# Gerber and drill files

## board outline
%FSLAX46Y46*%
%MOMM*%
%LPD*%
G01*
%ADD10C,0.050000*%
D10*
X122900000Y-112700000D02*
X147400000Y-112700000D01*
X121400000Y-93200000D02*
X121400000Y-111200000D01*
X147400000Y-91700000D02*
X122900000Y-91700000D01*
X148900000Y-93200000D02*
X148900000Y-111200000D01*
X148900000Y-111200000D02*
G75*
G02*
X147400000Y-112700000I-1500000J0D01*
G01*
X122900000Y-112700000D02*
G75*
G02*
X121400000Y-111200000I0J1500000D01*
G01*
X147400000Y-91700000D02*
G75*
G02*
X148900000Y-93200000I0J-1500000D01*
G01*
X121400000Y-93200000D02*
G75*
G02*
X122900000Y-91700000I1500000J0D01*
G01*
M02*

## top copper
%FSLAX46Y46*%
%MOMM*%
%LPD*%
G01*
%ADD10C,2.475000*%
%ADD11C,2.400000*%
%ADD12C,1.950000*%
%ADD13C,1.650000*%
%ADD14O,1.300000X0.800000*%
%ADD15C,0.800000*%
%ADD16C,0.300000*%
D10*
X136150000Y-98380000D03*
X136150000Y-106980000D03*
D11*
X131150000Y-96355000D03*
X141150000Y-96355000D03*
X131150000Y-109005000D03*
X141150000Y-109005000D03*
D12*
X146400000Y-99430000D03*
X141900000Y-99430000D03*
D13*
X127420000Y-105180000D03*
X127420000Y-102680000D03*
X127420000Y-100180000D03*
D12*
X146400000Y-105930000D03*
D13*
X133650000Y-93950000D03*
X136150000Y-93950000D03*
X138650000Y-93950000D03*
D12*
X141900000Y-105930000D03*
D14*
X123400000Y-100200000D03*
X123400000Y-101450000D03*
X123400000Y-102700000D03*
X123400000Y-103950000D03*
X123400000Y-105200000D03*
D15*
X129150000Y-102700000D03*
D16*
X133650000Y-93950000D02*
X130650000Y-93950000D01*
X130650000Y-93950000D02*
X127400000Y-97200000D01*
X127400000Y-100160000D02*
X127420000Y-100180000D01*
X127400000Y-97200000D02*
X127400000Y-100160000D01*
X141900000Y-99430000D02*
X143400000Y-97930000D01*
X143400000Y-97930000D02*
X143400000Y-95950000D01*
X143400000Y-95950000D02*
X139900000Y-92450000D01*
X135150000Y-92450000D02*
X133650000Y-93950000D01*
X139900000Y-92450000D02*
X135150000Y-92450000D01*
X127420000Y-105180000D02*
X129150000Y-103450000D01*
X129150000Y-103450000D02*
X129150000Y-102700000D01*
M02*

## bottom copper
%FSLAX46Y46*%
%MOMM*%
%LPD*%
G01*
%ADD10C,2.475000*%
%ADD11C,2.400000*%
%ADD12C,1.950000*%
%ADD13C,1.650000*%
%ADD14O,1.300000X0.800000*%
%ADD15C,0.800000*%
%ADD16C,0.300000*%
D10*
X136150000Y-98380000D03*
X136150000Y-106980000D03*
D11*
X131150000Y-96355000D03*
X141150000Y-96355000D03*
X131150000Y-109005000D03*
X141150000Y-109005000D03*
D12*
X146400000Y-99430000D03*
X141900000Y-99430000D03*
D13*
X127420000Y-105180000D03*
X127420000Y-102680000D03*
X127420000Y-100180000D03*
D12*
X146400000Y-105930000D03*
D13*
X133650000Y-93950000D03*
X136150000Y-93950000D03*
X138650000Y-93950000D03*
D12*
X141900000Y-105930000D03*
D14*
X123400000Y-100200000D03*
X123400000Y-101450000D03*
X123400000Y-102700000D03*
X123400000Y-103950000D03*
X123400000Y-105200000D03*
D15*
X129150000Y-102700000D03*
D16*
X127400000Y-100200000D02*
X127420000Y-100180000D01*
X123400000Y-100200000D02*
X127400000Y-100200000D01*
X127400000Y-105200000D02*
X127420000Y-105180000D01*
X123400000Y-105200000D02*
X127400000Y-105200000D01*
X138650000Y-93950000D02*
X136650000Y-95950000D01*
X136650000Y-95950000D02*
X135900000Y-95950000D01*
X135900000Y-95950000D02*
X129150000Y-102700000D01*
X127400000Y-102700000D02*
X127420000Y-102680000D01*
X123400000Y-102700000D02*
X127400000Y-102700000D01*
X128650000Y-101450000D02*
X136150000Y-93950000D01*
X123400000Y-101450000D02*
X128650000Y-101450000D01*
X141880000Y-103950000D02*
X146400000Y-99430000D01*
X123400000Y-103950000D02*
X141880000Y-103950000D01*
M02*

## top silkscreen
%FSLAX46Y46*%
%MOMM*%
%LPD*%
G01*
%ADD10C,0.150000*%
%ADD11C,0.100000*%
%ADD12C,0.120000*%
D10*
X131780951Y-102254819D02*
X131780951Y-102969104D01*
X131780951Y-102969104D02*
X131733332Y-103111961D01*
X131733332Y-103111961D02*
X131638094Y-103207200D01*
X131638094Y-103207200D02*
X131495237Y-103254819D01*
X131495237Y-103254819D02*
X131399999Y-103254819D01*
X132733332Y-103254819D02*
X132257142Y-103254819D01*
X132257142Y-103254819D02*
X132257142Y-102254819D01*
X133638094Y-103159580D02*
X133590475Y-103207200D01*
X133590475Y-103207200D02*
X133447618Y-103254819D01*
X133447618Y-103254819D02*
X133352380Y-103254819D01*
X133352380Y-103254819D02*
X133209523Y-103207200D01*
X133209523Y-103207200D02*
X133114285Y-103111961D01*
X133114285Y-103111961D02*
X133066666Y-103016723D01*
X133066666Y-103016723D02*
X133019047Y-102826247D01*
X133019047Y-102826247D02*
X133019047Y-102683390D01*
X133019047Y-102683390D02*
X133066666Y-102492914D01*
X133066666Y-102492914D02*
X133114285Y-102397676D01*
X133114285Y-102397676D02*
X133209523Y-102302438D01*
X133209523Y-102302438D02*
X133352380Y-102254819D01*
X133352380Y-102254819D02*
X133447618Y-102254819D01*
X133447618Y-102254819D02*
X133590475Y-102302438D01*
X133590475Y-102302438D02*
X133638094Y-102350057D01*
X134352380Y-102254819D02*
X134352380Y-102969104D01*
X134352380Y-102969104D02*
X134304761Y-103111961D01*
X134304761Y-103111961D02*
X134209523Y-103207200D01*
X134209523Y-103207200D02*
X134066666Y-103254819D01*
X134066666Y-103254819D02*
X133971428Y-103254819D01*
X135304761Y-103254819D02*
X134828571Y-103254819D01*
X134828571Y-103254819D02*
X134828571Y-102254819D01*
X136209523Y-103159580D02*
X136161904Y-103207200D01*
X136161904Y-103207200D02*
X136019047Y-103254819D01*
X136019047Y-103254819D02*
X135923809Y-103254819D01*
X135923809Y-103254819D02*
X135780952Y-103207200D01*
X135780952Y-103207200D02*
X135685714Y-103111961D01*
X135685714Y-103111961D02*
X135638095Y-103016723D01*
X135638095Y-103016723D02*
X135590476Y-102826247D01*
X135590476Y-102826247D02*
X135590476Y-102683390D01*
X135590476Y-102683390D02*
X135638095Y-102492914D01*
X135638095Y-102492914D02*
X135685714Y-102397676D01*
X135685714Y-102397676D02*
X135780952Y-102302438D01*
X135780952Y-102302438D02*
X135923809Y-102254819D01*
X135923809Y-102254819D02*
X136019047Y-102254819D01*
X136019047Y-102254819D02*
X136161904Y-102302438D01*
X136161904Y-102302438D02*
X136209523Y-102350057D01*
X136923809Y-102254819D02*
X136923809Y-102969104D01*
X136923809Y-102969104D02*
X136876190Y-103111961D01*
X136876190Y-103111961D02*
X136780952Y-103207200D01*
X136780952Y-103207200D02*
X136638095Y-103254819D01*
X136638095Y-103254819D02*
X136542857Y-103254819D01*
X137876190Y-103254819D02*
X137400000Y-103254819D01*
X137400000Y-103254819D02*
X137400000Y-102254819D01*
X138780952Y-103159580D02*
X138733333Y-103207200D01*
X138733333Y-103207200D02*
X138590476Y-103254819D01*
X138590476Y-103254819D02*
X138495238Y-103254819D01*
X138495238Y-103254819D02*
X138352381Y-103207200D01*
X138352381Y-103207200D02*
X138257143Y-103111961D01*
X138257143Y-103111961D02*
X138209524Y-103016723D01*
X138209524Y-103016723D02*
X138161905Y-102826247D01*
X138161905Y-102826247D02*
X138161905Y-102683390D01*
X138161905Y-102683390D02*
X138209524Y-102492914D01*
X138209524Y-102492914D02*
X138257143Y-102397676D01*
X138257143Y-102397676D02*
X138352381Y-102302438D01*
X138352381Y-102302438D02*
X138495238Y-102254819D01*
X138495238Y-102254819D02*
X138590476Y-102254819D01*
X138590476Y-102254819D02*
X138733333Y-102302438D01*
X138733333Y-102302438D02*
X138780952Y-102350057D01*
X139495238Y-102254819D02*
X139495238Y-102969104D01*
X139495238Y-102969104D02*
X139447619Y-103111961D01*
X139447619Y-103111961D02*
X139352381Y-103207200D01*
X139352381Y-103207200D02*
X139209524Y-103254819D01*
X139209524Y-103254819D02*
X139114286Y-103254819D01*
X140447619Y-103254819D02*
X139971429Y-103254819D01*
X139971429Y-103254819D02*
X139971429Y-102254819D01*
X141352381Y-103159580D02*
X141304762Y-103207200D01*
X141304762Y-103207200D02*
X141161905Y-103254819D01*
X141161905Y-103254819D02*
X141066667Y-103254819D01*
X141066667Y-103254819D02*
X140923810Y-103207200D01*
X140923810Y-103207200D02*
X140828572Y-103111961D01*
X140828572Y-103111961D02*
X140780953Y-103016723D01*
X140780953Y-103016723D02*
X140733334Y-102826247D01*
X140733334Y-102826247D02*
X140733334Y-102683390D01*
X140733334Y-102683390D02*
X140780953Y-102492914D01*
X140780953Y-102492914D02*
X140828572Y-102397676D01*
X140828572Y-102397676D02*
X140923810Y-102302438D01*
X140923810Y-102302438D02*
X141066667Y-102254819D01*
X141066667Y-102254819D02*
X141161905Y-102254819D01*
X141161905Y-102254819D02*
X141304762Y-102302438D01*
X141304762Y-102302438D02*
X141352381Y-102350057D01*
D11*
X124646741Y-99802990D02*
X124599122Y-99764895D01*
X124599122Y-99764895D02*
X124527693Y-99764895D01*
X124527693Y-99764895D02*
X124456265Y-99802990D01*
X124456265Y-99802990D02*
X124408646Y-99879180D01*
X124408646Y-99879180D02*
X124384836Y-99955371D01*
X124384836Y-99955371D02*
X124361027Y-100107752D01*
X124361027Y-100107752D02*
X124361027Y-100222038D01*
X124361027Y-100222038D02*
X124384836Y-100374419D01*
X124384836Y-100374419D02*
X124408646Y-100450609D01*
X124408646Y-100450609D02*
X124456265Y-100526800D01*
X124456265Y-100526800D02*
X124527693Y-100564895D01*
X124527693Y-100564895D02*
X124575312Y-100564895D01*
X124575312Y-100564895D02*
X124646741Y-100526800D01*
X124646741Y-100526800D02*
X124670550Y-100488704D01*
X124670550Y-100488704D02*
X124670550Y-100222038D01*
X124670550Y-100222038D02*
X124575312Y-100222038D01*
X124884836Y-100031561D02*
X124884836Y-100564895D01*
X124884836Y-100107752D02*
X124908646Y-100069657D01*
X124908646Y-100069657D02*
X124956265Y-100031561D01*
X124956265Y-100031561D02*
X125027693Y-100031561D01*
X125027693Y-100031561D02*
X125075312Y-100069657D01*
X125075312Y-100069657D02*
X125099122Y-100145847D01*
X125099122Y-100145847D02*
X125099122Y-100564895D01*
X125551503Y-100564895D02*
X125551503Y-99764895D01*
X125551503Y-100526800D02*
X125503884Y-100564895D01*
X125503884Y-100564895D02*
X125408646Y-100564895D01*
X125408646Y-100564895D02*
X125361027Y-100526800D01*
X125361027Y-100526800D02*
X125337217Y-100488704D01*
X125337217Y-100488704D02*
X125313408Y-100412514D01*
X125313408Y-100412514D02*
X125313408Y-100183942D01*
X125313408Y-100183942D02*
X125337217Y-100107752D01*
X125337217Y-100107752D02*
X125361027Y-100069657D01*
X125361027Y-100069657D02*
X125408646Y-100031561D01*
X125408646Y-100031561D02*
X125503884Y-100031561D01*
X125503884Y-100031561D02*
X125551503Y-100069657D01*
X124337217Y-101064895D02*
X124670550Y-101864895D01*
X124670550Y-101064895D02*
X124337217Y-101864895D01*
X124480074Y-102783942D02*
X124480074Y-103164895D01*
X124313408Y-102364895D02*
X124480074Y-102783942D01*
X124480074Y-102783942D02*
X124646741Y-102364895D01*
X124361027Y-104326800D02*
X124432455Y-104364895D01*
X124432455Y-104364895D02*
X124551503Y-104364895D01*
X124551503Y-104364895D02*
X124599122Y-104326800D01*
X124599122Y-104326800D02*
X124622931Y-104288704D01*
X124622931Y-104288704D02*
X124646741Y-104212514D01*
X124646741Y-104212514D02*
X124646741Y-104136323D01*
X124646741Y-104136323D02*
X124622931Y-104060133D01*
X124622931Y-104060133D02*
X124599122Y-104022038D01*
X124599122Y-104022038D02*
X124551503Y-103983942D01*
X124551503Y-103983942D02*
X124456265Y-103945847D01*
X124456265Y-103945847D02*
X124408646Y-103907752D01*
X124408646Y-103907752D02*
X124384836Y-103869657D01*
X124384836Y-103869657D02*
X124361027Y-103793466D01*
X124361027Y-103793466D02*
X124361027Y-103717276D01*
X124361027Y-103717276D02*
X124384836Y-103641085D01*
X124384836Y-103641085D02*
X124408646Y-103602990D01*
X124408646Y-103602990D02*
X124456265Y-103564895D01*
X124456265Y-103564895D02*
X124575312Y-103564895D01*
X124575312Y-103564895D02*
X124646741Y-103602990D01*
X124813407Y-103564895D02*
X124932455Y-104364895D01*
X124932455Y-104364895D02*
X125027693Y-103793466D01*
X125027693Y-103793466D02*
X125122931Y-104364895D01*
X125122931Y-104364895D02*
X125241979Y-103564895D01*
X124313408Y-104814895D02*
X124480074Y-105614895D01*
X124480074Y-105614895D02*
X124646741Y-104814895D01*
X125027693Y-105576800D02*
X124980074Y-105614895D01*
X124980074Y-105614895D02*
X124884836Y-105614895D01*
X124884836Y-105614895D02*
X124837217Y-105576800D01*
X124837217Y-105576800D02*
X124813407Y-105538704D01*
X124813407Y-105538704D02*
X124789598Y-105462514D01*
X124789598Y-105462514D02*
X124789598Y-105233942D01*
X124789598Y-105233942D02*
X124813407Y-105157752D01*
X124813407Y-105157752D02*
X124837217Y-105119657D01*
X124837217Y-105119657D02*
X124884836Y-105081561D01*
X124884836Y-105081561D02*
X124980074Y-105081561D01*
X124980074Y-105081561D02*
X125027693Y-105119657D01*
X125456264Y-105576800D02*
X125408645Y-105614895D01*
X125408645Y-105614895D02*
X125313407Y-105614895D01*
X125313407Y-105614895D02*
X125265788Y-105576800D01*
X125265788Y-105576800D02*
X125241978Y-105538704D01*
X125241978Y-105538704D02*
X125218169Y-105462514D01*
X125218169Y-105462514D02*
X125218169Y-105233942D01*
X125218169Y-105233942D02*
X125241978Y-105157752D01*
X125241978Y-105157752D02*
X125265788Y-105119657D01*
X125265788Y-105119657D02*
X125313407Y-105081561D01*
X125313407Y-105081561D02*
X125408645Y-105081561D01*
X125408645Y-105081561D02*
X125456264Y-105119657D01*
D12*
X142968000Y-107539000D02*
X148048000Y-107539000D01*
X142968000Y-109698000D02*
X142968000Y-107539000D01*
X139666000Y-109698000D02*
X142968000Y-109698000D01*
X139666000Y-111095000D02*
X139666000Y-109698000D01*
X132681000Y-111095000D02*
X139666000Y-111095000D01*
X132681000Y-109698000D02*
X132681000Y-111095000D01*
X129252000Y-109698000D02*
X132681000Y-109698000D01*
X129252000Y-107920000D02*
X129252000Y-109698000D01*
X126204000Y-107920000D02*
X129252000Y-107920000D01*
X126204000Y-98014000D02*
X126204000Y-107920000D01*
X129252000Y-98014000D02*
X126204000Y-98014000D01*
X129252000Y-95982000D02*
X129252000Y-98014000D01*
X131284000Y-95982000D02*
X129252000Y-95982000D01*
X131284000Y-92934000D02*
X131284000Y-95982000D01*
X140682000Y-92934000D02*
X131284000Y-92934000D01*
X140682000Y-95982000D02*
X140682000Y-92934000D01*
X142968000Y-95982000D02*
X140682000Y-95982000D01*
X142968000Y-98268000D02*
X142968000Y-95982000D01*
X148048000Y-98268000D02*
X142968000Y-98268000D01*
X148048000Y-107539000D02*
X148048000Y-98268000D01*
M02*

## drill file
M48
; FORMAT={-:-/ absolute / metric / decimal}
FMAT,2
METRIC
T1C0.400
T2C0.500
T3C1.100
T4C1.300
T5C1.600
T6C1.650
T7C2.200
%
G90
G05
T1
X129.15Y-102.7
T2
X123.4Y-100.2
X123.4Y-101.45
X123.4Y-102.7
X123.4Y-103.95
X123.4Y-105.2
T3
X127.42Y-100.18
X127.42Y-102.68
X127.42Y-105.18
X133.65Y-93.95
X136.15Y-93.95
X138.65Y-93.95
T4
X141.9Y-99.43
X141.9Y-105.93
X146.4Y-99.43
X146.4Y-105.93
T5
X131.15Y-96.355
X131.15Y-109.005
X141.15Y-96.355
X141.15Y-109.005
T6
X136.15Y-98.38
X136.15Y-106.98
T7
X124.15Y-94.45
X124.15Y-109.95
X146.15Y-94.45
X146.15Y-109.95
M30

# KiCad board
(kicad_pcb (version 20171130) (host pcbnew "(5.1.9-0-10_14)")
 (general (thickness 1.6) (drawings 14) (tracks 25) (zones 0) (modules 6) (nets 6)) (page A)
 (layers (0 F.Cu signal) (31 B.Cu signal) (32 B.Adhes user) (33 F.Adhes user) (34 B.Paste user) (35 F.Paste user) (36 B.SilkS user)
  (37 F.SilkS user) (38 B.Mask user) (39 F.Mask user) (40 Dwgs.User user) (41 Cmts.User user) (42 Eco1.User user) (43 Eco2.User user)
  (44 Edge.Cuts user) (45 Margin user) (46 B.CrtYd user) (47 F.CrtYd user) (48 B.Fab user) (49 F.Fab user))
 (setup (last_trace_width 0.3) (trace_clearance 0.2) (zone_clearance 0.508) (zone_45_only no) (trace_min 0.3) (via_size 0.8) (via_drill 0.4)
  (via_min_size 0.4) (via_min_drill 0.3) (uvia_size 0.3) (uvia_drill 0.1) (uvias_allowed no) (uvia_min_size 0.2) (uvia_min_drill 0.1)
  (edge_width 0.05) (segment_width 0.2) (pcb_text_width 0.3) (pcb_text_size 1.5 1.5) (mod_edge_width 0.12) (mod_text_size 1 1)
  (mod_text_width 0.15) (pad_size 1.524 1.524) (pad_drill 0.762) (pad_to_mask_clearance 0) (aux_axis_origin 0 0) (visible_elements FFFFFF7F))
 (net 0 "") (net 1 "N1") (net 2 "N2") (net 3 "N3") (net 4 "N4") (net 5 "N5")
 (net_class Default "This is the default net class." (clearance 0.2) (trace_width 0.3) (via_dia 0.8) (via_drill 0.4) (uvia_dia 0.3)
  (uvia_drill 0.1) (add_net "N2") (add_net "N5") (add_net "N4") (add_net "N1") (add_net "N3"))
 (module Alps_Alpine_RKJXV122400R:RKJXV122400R (layer F.Cu) (at 138.65 93.95 90)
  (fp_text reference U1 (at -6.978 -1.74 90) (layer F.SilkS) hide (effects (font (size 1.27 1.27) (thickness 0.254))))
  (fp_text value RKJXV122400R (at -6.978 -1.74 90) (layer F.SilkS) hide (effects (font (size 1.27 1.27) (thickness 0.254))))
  (fp_line (start -13.589 4.318) (end -13.589 9.398) (layer F.SilkS) (width 0.12))
  (fp_line (start -15.748 4.318) (end -13.589 4.318) (layer F.SilkS) (width 0.12))
  (fp_line (start -15.748 1.016) (end -15.748 4.318) (layer F.SilkS) (width 0.12))
  (fp_line (start -17.145 1.016) (end -15.748 1.016) (layer F.SilkS) (width 0.12))
  (fp_line (start -17.145 -5.969) (end -17.145 1.016) (layer F.SilkS) (width 0.12))
  (fp_line (start -15.748 -5.969) (end -17.145 -5.969) (layer F.SilkS) (width 0.12))
  (fp_line (start -15.748 -9.398) (end -15.748 -5.969) (layer F.SilkS) (width 0.12))
  (fp_line (start -13.97 -9.398) (end -15.748 -9.398) (layer F.SilkS) (width 0.12))
  (fp_line (start -13.97 -12.446) (end -13.97 -9.398) (layer F.SilkS) (width 0.12))
  (fp_line (start -4.064 -12.446) (end -13.97 -12.446) (layer F.SilkS) (width 0.12))
  (fp_line (start -4.064 -9.398) (end -4.064 -12.446) (layer F.SilkS) (width 0.12))
  (fp_line (start -2.032 -9.398) (end -4.064 -9.398) (layer F.SilkS) (width 0.12))
  (fp_line (start -2.032 -7.366) (end -2.032 -9.398) (layer F.SilkS) (width 0.12))
  (fp_line (start 1.016 -7.366) (end -2.032 -7.366) (layer F.SilkS) (width 0.12))
  (fp_line (start 1.016 2.032) (end 1.016 -7.366) (layer F.SilkS) (width 0.12))
  (fp_line (start -2.032 2.032) (end 1.016 2.032) (layer F.SilkS) (width 0.12))
  (fp_line (start -2.032 4.318) (end -2.032 2.032) (layer F.SilkS) (width 0.12))
  (fp_line (start -4.318 4.318) (end -2.032 4.318) (layer F.SilkS) (width 0.12))
  (fp_line (start -4.318 9.398) (end -4.318 4.318) (layer F.SilkS) (width 0.12))
  (fp_line (start -13.589 9.398) (end -4.318 9.398) (layer F.SilkS) (width 0.12))
  (pad MH6 thru_hole circle (at -4.43 -2.5 90) (size 2.475 2.475) (drill 1.65) (layers *.Cu *.Mask))
  (pad MH5 thru_hole circle (at -13.03 -2.5 90) (size 2.475 2.475) (drill 1.65) (layers *.Cu *.Mask))
  (pad MH4 thru_hole circle (at -2.405 -7.5 90) (size 2.4 2.4) (drill 1.6) (layers *.Cu *.Mask))
  (pad MH3 thru_hole circle (at -2.405 2.5 90) (size 2.4 2.4) (drill 1.6) (layers *.Cu *.Mask))
  (pad MH2 thru_hole circle (at -15.055 -7.5 90) (size 2.4 2.4) (drill 1.6) (layers *.Cu *.Mask))
  (pad MH1 thru_hole circle (at -15.055 2.5 90) (size 2.4 2.4) (drill 1.6) (layers *.Cu *.Mask))
  (pad D1 thru_hole circle (at -5.48 7.75 90) (size 1.95 1.95) (drill 1.3) (layers *.Cu *.Mask) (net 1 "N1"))
  (pad C1 thru_hole circle (at -5.48 3.25 90) (size 1.95 1.95) (drill 1.3) (layers *.Cu *.Mask) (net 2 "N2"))
  (pad B13 thru_hole circle (at -11.23 -11.23 90) (size 1.65 1.65) (drill 1.1) (layers *.Cu *.Mask) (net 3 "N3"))
  (pad B12 thru_hole circle (at -8.73 -11.23 90) (size 1.65 1.65) (drill 1.1) (layers *.Cu *.Mask) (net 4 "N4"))
  (pad B11 thru_hole circle (at -6.23 -11.23 90) (size 1.65 1.65) (drill 1.1) (layers *.Cu *.Mask) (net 2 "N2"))
  (pad B1 thru_hole circle (at -11.98 7.75 90) (size 1.95 1.95) (drill 1.3) (layers *.Cu *.Mask))
  (pad A13 thru_hole circle (at 0 -5 90) (size 1.65 1.65) (drill 1.1) (layers *.Cu *.Mask) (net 2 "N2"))
  (pad A12 thru_hole circle (at 0 -2.5 90) (size 1.65 1.65) (drill 1.1) (layers *.Cu *.Mask) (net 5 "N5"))
  (pad A11 thru_hole circle (at 0 0 90) (size 1.65 1.65) (drill 1.1) (layers *.Cu *.Mask) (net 3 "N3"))
  (pad A1 thru_hole circle (at -11.98 3.25 90) (size 1.95 1.95) (drill 1.3) (layers *.Cu *.Mask)))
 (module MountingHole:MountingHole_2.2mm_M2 (layer F.Cu) (at 146.15 109.95)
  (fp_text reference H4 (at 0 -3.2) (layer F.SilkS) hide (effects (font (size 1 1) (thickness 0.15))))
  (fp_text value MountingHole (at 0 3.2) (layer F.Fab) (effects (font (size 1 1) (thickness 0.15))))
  (pad 1 np_thru_hole circle (at 0 0) (size 2.2 2.2) (drill 2.2) (layers *.Cu *.Mask)))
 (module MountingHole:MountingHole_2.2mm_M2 (layer F.Cu) (at 146.15 94.45)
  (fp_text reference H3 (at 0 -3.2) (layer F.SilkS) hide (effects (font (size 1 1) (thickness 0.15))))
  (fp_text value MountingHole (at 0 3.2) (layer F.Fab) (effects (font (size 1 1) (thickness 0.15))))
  (pad 1 np_thru_hole circle (at 0 0) (size 2.2 2.2) (drill 2.2) (layers *.Cu *.Mask)))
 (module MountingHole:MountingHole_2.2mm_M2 (layer F.Cu) (at 124.15 109.95)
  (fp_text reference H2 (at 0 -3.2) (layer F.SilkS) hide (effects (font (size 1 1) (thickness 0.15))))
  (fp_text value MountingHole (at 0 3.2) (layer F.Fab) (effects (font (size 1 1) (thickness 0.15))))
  (pad 1 np_thru_hole circle (at 0 0) (size 2.2 2.2) (drill 2.2) (layers *.Cu *.Mask)))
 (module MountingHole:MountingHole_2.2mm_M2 (layer F.Cu) (at 124.15 94.45)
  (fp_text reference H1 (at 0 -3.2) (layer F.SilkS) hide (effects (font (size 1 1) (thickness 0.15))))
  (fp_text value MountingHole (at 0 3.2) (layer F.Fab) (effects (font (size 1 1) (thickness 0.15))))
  (pad 1 np_thru_hole circle (at 0 0) (size 2.2 2.2) (drill 2.2) (layers *.Cu *.Mask)))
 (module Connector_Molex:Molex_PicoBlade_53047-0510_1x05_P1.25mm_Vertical (layer B.Cu) (at 123.4 100.2 270)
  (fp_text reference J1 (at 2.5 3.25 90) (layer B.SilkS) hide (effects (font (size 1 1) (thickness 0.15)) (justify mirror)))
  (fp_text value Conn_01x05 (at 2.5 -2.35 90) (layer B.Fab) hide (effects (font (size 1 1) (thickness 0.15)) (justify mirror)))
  (pad 1 thru_hole oval (at 0 0 270) (size 0.8 1.3) (drill 0.5) (layers *.Cu *.Mask) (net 2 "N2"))
  (pad 2 thru_hole oval (at 1.25 0 270) (size 0.8 1.3) (drill 0.5) (layers *.Cu *.Mask) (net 5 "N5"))
  (pad 3 thru_hole oval (at 2.5 0 270) (size 0.8 1.3) (drill 0.5) (layers *.Cu *.Mask) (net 4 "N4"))
  (pad 4 thru_hole oval (at 3.75 0 270) (size 0.8 1.3) (drill 0.5) (layers *.Cu *.Mask) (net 1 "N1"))
  (pad 5 thru_hole oval (at 5 0 270) (size 0.8 1.3) (drill 0.5) (layers *.Cu *.Mask) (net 3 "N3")))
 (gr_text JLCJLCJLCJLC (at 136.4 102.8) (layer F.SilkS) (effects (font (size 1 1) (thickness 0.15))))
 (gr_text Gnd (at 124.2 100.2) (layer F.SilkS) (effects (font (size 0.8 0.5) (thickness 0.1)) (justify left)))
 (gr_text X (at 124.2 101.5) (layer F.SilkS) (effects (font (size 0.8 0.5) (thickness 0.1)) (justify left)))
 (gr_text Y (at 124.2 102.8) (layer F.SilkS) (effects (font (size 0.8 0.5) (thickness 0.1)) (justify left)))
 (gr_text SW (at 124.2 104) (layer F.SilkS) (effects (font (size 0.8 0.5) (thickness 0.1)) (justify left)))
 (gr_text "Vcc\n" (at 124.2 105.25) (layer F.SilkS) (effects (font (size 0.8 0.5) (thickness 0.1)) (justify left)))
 (gr_line (start 122.9 112.7) (end 147.4 112.7) (layer Edge.Cuts) (width 0.05))
 (gr_line (start 121.4 93.2) (end 121.4 111.2) (layer Edge.Cuts) (width 0.05))
 (gr_line (start 147.4 91.7) (end 122.9 91.7) (layer Edge.Cuts) (width 0.05))
 (gr_line (start 148.9 93.2) (end 148.9 111.2) (layer Edge.Cuts) (width 0.05))
 (gr_arc (start 147.4 111.2) (end 147.4 112.7) (angle -90) (layer Edge.Cuts) (width 0.05))
 (gr_arc (start 122.9 111.2) (end 121.4 111.2) (angle -90) (layer Edge.Cuts) (width 0.05))
 (gr_arc (start 147.4 93.2) (end 148.9 93.2) (angle -90) (layer Edge.Cuts) (width 0.05))
 (gr_arc (start 122.9 93.2) (end 122.9 91.7) (angle -90) (layer Edge.Cuts) (width 0.05))
 (segment (start 127.4 100.2) (end 127.42 100.18) (width 0.3) (layer B.Cu) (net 2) (status 30))
 (segment (start 123.4 100.2) (end 127.4 100.2) (width 0.3) (layer B.Cu) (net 2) (status 30))
 (segment (start 133.65 93.95) (end 130.65 93.95) (width 0.3) (layer F.Cu) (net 2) (status 10))
 (segment (start 130.65 93.95) (end 127.4 97.2) (width 0.3) (layer F.Cu) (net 2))
 (segment (start 127.4 100.16) (end 127.42 100.18) (width 0.3) (layer F.Cu) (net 2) (status 30))
 (segment (start 127.4 97.2) (end 127.4 100.16) (width 0.3) (layer F.Cu) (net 2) (status 20))
 (segment (start 141.9 99.43) (end 143.4 97.93) (width 0.3) (layer F.Cu) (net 2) (status 10))
 (segment (start 143.4 97.93) (end 143.4 95.95) (width 0.3) (layer F.Cu) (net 2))
 (segment (start 143.4 95.95) (end 139.9 92.45) (width 0.3) (layer F.Cu) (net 2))
 (segment (start 135.15 92.45) (end 133.65 93.95) (width 0.3) (layer F.Cu) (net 2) (status 20))
 (segment (start 139.9 92.45) (end 135.15 92.45) (width 0.3) (layer F.Cu) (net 2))
 (segment (start 127.4 105.2) (end 127.42 105.18) (width 0.3) (layer B.Cu) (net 3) (status 30))
 (segment (start 123.4 105.2) (end 127.4 105.2) (width 0.3) (layer B.Cu) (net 3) (status 30))
 (segment (start 127.42 105.18) (end 129.15 103.45) (width 0.3) (layer F.Cu) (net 3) (status 10))
 (segment (start 129.15 103.45) (end 129.15 102.7) (width 0.3) (layer F.Cu) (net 3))
 (via (at 129.15 102.7) (size 0.8) (drill 0.4) (layers F.Cu B.Cu) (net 3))
 (segment (start 138.65 93.95) (end 136.65 95.95) (width 0.3) (layer B.Cu) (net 3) (status 10))
 (segment (start 136.65 95.95) (end 135.9 95.95) (width 0.3) (layer B.Cu) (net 3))
 (segment (start 135.9 95.95) (end 129.15 102.7) (width 0.3) (layer B.Cu) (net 3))
 (segment (start 127.4 102.7) (end 127.42 102.68) (width 0.3) (layer B.Cu) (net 4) (status 30))
 (segment (start 123.4 102.7) (end 127.4 102.7) (width 0.3) (layer B.Cu) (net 4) (status 30))
 (segment (start 128.65 101.45) (end 136.15 93.95) (width 0.3) (layer B.Cu) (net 5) (status 20))
 (segment (start 123.4 101.45) (end 128.65 101.45) (width 0.3) (layer B.Cu) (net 5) (status 10))
 (segment (start 141.88 103.95) (end 146.4 99.43) (width 0.3) (layer B.Cu) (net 1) (status 20))
 (segment (start 123.4 103.95) (end 141.88 103.95) (width 0.3) (layer B.Cu) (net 1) (status 10)))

